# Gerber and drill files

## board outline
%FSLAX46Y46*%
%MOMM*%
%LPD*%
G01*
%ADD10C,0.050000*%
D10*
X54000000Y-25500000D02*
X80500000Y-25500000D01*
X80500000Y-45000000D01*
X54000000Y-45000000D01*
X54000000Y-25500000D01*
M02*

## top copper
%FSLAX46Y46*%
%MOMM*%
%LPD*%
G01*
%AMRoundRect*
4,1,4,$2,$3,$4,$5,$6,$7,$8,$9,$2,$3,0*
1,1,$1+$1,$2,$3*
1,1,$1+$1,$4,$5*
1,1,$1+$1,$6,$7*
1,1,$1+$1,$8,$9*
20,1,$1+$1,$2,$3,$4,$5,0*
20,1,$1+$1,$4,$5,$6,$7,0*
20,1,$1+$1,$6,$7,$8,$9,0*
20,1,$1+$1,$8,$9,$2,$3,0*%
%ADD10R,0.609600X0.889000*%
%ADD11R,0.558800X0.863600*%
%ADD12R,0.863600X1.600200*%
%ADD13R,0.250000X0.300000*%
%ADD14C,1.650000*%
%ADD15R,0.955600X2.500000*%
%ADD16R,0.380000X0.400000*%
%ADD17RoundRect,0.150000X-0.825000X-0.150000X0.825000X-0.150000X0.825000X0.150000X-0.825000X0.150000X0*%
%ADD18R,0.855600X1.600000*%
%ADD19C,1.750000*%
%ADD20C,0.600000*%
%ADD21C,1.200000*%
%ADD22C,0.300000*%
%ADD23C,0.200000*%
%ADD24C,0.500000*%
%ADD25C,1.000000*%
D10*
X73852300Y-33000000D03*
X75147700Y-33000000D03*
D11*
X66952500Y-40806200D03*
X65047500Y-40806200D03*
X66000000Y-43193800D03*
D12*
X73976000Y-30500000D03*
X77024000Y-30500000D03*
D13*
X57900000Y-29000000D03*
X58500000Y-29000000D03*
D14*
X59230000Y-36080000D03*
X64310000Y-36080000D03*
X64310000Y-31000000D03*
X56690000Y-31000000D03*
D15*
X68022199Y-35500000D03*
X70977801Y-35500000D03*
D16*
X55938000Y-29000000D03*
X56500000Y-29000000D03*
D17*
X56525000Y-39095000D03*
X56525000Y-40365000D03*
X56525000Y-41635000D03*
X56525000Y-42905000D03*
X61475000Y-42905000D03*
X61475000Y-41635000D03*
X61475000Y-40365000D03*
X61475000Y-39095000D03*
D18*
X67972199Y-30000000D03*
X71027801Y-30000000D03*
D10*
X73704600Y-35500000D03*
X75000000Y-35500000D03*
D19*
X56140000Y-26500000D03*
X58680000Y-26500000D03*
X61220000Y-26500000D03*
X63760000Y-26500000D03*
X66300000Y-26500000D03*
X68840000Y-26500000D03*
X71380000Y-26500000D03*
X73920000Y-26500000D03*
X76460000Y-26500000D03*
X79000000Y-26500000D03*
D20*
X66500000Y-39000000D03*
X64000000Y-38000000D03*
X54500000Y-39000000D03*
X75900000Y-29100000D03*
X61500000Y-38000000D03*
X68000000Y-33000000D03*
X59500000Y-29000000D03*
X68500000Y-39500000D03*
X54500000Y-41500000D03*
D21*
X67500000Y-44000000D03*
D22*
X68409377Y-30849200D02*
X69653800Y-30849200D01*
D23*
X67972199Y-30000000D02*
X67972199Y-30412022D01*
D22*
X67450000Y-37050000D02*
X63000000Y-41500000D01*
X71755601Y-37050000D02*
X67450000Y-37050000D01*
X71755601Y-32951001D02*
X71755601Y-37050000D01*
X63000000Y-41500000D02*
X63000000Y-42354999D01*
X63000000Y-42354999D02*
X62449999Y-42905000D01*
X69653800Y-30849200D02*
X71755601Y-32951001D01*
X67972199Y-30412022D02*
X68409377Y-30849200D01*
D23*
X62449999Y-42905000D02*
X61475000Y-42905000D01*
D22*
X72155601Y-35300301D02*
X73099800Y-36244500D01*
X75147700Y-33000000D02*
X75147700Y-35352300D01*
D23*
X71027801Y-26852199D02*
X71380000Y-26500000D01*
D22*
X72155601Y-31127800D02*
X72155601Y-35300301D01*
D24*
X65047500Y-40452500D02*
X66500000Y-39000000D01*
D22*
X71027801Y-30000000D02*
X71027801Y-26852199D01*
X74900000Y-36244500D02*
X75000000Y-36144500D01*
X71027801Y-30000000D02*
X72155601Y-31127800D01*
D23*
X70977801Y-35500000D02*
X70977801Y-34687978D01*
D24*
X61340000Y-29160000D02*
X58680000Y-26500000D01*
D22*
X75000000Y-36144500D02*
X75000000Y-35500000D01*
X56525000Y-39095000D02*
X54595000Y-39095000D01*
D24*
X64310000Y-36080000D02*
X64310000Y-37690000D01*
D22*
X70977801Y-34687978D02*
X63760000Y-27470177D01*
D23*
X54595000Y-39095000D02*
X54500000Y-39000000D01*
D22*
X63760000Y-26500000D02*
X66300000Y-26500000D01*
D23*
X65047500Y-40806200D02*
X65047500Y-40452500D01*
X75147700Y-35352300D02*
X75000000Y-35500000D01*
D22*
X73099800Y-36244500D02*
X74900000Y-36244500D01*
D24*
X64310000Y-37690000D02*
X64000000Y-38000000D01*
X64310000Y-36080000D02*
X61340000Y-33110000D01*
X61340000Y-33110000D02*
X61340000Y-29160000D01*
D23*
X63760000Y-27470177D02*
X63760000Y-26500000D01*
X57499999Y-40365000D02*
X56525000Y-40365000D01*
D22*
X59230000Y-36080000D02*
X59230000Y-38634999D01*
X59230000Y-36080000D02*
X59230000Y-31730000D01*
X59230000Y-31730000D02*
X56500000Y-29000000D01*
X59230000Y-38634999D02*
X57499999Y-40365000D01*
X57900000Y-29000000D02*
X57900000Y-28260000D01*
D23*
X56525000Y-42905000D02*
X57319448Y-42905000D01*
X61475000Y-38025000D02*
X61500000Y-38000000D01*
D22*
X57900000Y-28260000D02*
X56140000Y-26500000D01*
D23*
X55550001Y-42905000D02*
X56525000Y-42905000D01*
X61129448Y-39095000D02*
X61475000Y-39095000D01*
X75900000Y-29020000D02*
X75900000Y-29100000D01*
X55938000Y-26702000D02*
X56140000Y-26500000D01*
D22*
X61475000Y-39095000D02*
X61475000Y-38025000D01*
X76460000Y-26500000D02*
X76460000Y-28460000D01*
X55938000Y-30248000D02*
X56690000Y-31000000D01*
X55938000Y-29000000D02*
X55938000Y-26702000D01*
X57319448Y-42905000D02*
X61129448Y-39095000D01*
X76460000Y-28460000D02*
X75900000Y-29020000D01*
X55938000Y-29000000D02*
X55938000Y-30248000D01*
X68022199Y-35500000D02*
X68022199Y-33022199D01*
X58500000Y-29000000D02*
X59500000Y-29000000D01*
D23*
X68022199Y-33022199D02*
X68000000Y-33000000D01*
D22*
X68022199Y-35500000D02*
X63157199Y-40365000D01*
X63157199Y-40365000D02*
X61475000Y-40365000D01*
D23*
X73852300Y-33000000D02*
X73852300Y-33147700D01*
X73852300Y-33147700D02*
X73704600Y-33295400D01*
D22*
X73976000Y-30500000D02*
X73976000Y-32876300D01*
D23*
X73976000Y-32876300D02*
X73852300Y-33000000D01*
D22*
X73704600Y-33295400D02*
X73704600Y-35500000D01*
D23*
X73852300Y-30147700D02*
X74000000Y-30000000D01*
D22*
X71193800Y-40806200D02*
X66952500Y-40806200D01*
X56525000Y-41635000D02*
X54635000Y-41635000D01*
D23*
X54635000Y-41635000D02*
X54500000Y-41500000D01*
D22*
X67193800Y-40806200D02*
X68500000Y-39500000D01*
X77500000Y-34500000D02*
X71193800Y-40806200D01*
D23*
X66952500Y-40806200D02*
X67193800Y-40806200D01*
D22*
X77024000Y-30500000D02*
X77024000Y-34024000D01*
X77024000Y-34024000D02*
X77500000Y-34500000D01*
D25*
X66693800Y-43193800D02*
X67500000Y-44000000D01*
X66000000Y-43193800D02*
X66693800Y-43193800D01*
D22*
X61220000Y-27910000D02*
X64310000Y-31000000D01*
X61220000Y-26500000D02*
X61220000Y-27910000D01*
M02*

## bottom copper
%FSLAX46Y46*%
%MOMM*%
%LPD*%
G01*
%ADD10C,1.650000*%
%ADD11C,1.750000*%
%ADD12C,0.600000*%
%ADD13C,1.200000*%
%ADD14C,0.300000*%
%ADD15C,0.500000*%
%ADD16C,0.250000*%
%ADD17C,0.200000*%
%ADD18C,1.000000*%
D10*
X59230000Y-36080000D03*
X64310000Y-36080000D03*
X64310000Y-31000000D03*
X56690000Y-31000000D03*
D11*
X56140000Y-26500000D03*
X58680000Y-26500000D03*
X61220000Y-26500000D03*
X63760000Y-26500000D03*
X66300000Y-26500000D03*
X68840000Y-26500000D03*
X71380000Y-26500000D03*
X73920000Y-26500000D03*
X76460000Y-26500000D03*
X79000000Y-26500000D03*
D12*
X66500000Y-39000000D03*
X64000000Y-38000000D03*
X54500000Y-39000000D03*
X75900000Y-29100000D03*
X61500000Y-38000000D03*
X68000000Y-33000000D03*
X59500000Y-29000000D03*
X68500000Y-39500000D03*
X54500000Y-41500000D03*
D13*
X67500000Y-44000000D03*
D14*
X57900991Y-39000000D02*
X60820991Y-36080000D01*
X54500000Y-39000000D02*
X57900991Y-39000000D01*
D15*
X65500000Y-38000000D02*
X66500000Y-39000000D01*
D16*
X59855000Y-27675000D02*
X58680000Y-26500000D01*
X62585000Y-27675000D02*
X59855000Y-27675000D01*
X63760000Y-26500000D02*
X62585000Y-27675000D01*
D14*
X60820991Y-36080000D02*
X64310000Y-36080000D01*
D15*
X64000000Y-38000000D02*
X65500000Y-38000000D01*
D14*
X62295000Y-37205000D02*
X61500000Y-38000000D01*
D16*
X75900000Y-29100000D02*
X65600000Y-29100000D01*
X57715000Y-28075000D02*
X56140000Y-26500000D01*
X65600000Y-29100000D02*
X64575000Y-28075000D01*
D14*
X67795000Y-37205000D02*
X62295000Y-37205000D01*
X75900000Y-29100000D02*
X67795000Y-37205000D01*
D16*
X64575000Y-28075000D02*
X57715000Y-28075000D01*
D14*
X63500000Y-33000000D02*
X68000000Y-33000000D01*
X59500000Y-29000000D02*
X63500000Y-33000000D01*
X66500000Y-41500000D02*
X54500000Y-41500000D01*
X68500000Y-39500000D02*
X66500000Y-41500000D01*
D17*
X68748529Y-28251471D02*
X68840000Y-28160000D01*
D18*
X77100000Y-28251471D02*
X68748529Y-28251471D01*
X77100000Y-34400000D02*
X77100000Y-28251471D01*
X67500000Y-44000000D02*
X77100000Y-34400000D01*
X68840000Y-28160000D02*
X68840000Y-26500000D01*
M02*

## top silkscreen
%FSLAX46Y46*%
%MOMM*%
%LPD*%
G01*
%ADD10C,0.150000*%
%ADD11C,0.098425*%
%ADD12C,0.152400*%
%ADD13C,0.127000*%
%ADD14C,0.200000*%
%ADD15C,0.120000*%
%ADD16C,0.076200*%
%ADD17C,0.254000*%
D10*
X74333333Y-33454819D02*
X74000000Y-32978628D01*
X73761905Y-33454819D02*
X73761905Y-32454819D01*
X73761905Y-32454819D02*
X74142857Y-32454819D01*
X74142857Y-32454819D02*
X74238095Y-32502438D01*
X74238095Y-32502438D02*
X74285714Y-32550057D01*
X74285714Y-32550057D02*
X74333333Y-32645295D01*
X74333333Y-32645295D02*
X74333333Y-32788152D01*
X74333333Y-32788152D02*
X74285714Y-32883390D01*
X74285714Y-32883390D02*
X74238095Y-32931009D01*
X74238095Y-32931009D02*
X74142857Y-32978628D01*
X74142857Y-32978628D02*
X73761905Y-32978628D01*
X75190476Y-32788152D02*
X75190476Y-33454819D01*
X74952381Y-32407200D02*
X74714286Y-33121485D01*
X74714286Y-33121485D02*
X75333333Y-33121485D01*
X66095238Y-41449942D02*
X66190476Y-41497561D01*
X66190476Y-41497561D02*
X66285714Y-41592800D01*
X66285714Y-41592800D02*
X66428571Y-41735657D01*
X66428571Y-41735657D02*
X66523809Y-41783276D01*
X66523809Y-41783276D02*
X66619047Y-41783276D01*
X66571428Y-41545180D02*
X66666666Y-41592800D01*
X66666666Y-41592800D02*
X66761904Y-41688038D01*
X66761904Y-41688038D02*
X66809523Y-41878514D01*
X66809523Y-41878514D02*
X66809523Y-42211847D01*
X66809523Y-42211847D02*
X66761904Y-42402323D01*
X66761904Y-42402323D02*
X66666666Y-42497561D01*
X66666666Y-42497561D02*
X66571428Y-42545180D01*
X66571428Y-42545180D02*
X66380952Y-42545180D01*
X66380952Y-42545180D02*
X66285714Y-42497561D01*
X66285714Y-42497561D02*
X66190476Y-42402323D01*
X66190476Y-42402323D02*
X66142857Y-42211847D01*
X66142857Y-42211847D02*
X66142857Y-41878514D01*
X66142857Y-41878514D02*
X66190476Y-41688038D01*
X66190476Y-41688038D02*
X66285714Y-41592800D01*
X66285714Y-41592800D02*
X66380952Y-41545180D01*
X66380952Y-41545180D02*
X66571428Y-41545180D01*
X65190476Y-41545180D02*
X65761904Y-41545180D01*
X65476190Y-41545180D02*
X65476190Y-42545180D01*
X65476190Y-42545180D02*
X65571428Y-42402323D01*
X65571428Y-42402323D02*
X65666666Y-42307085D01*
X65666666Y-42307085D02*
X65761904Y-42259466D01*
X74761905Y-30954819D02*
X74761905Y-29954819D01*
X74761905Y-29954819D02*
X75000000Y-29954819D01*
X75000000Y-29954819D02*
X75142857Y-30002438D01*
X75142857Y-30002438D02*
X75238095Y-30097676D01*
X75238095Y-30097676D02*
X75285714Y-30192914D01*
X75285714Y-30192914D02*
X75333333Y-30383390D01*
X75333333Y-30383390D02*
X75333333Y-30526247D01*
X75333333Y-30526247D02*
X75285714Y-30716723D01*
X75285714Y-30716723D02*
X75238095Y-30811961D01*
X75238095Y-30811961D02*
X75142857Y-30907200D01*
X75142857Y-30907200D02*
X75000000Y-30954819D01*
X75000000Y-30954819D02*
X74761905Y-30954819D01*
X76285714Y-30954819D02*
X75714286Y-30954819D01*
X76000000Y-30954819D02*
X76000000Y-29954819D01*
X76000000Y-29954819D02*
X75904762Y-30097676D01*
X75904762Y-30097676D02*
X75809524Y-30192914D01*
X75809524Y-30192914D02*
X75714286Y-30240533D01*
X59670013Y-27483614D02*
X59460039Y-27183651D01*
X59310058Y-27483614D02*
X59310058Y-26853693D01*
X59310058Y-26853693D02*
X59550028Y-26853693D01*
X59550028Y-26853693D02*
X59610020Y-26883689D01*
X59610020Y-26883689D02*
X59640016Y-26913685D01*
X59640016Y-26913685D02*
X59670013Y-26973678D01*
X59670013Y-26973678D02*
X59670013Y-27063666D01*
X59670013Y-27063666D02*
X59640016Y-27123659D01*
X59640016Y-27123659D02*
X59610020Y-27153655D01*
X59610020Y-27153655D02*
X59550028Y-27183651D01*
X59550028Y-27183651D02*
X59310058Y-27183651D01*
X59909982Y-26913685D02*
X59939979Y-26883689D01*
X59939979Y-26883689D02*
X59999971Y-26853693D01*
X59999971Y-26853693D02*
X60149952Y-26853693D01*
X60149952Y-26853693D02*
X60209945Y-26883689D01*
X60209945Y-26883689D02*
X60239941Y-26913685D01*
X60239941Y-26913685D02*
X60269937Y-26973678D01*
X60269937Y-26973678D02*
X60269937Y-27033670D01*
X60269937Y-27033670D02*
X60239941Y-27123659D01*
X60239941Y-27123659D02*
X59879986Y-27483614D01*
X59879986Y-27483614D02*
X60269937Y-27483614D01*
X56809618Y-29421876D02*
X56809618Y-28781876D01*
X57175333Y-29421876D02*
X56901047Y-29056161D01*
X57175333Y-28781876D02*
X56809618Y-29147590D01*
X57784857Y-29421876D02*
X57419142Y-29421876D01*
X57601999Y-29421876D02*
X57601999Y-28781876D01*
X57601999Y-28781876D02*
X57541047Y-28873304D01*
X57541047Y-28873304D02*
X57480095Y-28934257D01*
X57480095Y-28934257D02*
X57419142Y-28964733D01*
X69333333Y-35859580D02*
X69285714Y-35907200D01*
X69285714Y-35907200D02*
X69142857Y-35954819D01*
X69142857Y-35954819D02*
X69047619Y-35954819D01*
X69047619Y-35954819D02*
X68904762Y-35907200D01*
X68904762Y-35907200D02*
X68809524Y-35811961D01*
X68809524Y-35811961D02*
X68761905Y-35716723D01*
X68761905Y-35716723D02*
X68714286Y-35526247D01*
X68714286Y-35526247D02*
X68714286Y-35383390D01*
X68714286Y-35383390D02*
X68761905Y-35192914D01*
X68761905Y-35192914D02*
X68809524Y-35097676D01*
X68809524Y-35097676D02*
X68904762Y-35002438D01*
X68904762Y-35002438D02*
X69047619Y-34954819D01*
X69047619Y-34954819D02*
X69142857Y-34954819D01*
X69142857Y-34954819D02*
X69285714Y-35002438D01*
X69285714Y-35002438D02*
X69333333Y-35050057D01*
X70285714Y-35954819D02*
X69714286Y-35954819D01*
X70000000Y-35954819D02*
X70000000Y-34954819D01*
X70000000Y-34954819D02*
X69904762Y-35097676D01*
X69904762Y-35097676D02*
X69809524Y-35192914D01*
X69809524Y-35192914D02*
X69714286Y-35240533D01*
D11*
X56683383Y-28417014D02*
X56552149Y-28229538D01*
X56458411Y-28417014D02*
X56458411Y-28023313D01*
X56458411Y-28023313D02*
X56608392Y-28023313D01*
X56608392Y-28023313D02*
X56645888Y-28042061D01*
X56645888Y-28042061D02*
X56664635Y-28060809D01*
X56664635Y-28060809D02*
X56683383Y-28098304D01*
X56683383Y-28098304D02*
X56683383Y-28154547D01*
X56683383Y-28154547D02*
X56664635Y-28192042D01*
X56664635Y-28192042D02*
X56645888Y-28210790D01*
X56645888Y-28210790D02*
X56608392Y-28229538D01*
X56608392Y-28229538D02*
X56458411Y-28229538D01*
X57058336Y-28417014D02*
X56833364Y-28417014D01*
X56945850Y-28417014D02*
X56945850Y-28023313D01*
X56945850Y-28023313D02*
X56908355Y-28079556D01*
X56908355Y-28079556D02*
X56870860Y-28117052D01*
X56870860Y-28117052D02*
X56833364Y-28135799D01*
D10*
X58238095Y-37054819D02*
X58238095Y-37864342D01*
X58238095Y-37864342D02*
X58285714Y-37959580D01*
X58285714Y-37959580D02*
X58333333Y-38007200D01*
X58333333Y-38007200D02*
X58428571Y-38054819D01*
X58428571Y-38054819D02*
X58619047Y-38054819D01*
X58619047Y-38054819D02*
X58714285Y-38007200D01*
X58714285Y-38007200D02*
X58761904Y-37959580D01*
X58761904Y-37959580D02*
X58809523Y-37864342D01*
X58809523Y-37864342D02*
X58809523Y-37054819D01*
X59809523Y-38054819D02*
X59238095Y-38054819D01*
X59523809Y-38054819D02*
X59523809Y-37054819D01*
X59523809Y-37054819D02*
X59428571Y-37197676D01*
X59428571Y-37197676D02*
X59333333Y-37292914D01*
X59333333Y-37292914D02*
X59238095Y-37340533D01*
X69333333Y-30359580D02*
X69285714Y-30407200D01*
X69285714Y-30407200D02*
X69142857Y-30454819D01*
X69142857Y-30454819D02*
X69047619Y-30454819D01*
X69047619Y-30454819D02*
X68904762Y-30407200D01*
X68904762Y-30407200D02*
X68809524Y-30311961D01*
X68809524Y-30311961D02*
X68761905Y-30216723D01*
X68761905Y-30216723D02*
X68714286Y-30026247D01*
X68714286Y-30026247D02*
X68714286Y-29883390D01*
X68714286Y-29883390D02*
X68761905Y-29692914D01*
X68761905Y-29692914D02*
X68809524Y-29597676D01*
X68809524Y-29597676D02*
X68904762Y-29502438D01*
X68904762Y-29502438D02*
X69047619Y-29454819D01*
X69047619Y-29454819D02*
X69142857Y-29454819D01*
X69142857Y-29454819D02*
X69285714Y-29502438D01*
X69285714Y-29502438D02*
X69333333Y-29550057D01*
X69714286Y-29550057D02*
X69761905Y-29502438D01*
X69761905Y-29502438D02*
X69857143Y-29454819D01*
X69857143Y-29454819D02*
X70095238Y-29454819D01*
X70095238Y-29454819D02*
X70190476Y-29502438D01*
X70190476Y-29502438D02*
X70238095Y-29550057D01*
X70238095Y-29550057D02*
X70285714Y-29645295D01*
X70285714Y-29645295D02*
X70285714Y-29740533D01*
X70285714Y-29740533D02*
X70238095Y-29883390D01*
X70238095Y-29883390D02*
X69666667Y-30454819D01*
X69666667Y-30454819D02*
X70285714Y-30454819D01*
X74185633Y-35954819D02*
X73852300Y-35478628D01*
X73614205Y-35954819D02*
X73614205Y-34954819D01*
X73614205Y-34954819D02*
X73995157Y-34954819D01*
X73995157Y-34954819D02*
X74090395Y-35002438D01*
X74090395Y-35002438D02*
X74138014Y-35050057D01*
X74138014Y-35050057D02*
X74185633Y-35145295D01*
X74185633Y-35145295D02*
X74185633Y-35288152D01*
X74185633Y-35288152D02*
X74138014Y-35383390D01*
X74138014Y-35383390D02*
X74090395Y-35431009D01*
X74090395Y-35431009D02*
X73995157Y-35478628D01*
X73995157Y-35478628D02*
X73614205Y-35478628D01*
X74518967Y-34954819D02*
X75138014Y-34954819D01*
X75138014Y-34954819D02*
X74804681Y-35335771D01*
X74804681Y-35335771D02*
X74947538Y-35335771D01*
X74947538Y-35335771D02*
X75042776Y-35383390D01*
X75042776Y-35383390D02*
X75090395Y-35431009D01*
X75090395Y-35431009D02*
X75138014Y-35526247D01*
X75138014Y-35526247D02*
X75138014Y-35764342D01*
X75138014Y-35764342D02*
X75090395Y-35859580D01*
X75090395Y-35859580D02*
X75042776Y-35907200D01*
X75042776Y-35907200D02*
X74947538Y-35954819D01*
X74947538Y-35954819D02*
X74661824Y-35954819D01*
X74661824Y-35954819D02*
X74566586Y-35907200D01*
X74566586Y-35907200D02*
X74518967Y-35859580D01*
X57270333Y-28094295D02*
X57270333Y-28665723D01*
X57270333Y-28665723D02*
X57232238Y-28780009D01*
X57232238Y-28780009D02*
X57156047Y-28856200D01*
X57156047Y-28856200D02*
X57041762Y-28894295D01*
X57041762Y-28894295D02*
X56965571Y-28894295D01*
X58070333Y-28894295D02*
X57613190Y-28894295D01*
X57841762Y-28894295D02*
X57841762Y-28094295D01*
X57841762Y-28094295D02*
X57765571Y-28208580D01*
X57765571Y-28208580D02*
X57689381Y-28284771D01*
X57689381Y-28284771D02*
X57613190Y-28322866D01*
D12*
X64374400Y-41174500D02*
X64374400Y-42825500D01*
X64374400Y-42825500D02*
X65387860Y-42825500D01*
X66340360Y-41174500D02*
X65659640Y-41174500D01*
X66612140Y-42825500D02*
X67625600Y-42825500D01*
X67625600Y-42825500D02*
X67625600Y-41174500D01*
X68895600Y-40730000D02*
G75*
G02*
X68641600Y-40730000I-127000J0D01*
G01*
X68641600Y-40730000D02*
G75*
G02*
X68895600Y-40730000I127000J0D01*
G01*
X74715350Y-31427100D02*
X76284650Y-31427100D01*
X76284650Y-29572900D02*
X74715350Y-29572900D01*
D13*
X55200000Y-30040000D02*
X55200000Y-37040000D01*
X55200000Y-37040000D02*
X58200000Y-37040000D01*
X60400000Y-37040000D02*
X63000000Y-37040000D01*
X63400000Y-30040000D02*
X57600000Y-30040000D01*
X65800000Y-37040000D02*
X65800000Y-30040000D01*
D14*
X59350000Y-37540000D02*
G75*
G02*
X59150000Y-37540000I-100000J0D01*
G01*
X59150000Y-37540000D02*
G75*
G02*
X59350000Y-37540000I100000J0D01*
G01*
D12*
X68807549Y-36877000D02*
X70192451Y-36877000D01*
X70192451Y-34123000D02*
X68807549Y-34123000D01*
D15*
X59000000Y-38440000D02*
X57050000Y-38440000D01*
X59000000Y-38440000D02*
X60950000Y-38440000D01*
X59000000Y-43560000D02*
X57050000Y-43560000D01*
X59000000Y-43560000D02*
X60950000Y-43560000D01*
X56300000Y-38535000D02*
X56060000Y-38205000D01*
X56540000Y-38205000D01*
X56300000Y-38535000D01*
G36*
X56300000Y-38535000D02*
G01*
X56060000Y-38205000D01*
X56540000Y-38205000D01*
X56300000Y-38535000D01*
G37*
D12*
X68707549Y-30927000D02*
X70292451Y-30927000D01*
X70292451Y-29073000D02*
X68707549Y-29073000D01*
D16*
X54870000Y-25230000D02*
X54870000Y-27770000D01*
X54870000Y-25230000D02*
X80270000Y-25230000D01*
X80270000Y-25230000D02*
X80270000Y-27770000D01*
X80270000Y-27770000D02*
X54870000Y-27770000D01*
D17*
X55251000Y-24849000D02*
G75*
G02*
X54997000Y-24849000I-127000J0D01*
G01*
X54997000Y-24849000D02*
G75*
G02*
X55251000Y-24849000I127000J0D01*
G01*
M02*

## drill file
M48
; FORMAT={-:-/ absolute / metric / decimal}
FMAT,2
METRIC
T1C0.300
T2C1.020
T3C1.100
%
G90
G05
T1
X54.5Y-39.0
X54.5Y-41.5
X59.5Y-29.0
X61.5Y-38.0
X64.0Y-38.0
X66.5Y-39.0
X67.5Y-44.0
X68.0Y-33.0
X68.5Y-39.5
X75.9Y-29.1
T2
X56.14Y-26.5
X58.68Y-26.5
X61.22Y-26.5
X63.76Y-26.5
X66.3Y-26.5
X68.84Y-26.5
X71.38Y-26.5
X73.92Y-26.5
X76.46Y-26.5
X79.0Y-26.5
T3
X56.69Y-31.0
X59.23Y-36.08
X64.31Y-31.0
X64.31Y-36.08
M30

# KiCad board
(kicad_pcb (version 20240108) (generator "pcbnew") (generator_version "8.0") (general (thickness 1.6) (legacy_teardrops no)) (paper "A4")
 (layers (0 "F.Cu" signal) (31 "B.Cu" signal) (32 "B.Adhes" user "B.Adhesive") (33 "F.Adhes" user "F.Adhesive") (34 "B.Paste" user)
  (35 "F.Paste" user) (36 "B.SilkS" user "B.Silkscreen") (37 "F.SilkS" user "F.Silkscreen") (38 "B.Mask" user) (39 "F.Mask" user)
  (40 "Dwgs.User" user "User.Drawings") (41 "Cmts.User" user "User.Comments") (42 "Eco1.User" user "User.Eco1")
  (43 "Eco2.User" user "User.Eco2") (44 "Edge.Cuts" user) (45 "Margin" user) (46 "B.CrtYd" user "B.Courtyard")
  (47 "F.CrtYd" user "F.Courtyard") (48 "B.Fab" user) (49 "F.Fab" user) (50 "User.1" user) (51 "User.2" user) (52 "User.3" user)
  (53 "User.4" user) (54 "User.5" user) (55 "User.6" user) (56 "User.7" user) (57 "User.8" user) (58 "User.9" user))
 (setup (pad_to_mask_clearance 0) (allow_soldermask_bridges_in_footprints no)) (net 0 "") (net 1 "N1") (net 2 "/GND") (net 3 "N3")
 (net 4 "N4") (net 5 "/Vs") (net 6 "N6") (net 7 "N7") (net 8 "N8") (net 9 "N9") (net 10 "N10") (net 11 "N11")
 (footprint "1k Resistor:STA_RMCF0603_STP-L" (layer "F.Cu") (at 74.5 33)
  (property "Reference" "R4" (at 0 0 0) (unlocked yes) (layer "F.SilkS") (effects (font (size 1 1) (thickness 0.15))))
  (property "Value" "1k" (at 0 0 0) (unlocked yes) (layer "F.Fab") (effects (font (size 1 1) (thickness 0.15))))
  (pad "1" smd rect (at -0.6477 0) (size 0.6096 0.889) (layers "F.Cu" "F.Paste" "F.Mask") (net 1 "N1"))
  (pad "2" smd rect (at 0.6477 0) (size 0.6096 0.889) (layers "F.Cu" "F.Paste" "F.Mask") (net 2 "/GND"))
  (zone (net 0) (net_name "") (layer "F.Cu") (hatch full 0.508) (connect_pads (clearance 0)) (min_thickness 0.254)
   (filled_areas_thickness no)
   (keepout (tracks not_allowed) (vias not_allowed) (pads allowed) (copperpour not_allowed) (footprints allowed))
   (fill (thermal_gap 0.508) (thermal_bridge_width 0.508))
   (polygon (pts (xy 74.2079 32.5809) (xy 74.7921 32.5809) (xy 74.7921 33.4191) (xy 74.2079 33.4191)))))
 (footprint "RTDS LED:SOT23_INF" (layer "F.Cu") (at 66 42 180)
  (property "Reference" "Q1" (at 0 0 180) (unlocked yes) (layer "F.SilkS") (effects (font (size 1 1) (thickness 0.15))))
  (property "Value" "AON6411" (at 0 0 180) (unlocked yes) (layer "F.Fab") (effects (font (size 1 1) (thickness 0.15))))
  (fp_line (start 1.6256 0.8255) (end 1.6256 -0.8255) (stroke (width 0.1524) (type solid)) (layer "F.SilkS"))
  (fp_line (start 1.6256 -0.8255) (end 0.61214 -0.8255) (stroke (width 0.1524) (type solid)) (layer "F.SilkS"))
  (fp_line (start -0.34036 0.8255) (end 0.34036 0.8255) (stroke (width 0.1524) (type solid)) (layer "F.SilkS"))
  (fp_line (start -0.61214 -0.8255) (end -1.6256 -0.8255) (stroke (width 0.1524) (type solid)) (layer "F.SilkS"))
  (fp_line (start -1.6256 -0.8255) (end -1.6256 0.8255) (stroke (width 0.1524) (type solid)) (layer "F.SilkS"))
  (fp_circle (center -2.7686 1.27) (end -2.6416 1.27) (stroke (width 0.1524) (type solid)) (fill none) (layer "F.SilkS"))
  (pad "1" smd rect (at -0.9525 1.1938 180) (size 0.5588 0.8636) (layers "F.Cu" "F.Paste" "F.Mask") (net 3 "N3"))
  (pad "2" smd rect (at 0.9525 1.1938 180) (size 0.5588 0.8636) (layers "F.Cu" "F.Paste" "F.Mask") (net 2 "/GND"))
  (pad "3" smd rect (at 0 -1.1938 180) (size 0.5588 0.8636) (layers "F.Cu" "F.Paste" "F.Mask") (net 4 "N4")))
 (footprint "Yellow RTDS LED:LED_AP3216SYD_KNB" (layer "F.Cu") (at 75.5 30.5)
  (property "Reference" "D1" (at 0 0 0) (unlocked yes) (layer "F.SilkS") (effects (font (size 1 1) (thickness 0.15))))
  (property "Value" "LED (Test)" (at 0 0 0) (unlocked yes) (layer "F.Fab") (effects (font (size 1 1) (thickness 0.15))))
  (fp_line (start -0.78465 0.9271) (end 0.78465 0.9271) (stroke (width 0.1524) (type solid)) (layer "F.SilkS"))
  (fp_line (start 0.78465 -0.9271) (end -0.78465 -0.9271) (stroke (width 0.1524) (type solid)) (layer "F.SilkS"))
  (pad "1" smd rect (at -1.524 0) (size 0.8636 1.6002) (layers "F.Cu" "F.Paste" "F.Mask") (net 1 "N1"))
  (pad "2" smd rect (at 1.524 0) (size 0.8636 1.6002) (layers "F.Cu" "F.Paste" "F.Mask") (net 3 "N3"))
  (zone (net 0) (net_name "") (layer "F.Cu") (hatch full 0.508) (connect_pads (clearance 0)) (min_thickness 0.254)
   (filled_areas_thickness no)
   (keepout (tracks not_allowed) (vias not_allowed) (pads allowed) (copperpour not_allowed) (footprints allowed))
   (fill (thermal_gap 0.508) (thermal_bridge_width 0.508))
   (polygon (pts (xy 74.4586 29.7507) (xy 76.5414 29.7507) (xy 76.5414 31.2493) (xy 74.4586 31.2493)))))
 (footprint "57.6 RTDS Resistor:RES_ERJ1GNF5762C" (layer "F.Cu") (at 58.2 29)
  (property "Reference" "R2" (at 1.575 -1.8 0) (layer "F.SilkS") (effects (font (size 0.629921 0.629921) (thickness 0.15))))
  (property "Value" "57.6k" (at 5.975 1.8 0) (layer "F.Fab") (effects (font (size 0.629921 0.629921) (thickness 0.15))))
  (pad "1" smd rect (at -0.3 0) (size 0.25 0.3) (layers "F.Cu" "F.Paste" "F.Mask") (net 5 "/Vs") (solder_mask_margin 0.102))
  (pad "2" smd rect (at 0.3 0) (size 0.25 0.3) (layers "F.Cu" "F.Paste" "F.Mask") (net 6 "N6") (solder_mask_margin 0.102)))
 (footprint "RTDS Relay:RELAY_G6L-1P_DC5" (layer "F.Cu") (at 60.5 33.54)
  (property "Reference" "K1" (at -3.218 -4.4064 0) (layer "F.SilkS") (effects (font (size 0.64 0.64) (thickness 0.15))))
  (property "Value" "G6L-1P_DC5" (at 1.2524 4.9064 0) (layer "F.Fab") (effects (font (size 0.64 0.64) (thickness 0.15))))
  (fp_line (start -5.3 -3.5) (end -5.3 3.5) (stroke (width 0.127) (type solid)) (layer "F.SilkS"))
  (fp_line (start -5.3 3.5) (end -2.3 3.5) (stroke (width 0.127) (type solid)) (layer "F.SilkS"))
  (fp_line (start -0.1 3.5) (end 2.5 3.5) (stroke (width 0.127) (type solid)) (layer "F.SilkS"))
  (fp_line (start 2.9 -3.5) (end -2.9 -3.5) (stroke (width 0.127) (type solid)) (layer "F.SilkS"))
  (fp_line (start 5.3 3.5) (end 5.3 -3.5) (stroke (width 0.127) (type solid)) (layer "F.SilkS"))
  (fp_circle (center -1.25 4) (end -1.15 4) (stroke (width 0.2) (type solid)) (fill none) (layer "F.SilkS"))
  (pad "2" thru_hole circle (at -1.27 2.54) (size 1.65 1.65) (drill 1.1) (layers "*.Cu" "*.Mask") (remove_unused_layers no) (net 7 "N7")
   (solder_mask_margin 0.102))
  (pad "4" thru_hole circle (at 3.81 2.54) (size 1.65 1.65) (drill 1.1) (layers "*.Cu" "*.Mask") (remove_unused_layers no) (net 2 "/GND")
   (solder_mask_margin 0.102))
  (pad "5" thru_hole circle (at 3.81 -2.54) (size 1.65 1.65) (drill 1.1) (layers "*.Cu" "*.Mask") (remove_unused_layers no) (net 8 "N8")
   (solder_mask_margin 0.102))
  (pad "8" thru_hole circle (at -3.81 -2.54) (size 1.65 1.65) (drill 1.1) (layers "*.Cu" "*.Mask") (remove_unused_layers no) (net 5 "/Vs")
   (solder_mask_margin 0.102)))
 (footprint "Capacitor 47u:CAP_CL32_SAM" (layer "F.Cu") (at 69.5 35.5)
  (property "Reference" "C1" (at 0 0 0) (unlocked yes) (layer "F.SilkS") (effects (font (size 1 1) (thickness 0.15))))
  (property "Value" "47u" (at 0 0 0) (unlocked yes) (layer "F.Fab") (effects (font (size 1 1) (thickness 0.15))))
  (fp_line (start -0.692451 1.377) (end 0.692451 1.377) (stroke (width 0.1524) (type solid)) (layer "F.SilkS"))
  (fp_line (start 0.692451 -1.377) (end -0.692451 -1.377) (stroke (width 0.1524) (type solid)) (layer "F.SilkS"))
  (pad "1" smd rect (at -1.477801 0) (size 0.9556 2.5) (layers "F.Cu" "F.Paste" "F.Mask") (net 6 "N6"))
  (pad "2" smd rect (at 1.477801 0) (size 0.9556 2.5) (layers "F.Cu" "F.Paste" "F.Mask") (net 2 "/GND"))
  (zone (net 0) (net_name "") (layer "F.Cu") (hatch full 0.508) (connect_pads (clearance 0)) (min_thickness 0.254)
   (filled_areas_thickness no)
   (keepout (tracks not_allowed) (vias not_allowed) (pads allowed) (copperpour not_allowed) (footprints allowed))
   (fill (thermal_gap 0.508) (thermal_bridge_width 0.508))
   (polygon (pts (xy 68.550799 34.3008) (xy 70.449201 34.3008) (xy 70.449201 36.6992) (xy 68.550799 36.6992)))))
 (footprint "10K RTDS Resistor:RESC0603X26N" (layer "F.Cu") (at 56.219 29)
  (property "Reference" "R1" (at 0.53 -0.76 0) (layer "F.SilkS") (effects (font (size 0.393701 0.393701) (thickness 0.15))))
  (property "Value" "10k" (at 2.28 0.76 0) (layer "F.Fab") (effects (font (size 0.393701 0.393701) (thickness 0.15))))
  (pad "1" smd rect (at -0.281 0) (size 0.38 0.4) (layers "F.Cu" "F.Paste" "F.Mask") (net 5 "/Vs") (solder_mask_margin 0.102))
  (pad "2" smd rect (at 0.281 0) (size 0.38 0.4) (layers "F.Cu" "F.Paste" "F.Mask") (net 7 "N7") (solder_mask_margin 0.102)))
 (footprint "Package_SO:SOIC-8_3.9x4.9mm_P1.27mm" (layer "F.Cu") (at 59 41)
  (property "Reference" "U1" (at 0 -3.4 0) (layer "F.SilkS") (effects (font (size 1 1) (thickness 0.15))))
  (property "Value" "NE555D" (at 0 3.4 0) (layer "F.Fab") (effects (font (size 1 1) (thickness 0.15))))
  (fp_line (start 0 -2.56) (end -1.95 -2.56) (stroke (width 0.12) (type solid)) (layer "F.SilkS"))
  (fp_line (start 0 -2.56) (end 1.95 -2.56) (stroke (width 0.12) (type solid)) (layer "F.SilkS"))
  (fp_line (start 0 2.56) (end -1.95 2.56) (stroke (width 0.12) (type solid)) (layer "F.SilkS"))
  (fp_line (start 0 2.56) (end 1.95 2.56) (stroke (width 0.12) (type solid)) (layer "F.SilkS"))
  (fp_poly
   (pts (xy -2.7 -2.465) (xy -2.94 -2.795) (xy -2.46 -2.795) (xy -2.7 -2.465)) (stroke (width 0.12) (type solid)) (fill solid)
   (layer "F.SilkS"))
  (pad "1" smd roundrect (at -2.475 -1.905) (size 1.95 0.6) (layers "F.Cu" "F.Paste" "F.Mask") (roundrect_rratio 0.25) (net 2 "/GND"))
  (pad "2" smd roundrect (at -2.475 -0.635) (size 1.95 0.6) (layers "F.Cu" "F.Paste" "F.Mask") (roundrect_rratio 0.25) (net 7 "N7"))
  (pad "3" smd roundrect (at -2.475 0.635) (size 1.95 0.6) (layers "F.Cu" "F.Paste" "F.Mask") (roundrect_rratio 0.25) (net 3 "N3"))
  (pad "4" smd roundrect (at -2.475 1.905) (size 1.95 0.6) (layers "F.Cu" "F.Paste" "F.Mask") (roundrect_rratio 0.25) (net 5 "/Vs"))
  (pad "5" smd roundrect (at 2.475 1.905) (size 1.95 0.6) (layers "F.Cu" "F.Paste" "F.Mask") (roundrect_rratio 0.25) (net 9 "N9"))
  (pad "6" smd roundrect (at 2.475 0.635) (size 1.95 0.6) (layers "F.Cu" "F.Paste" "F.Mask") (roundrect_rratio 0.25) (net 6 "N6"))
  (pad "7" smd roundrect (at 2.475 -0.635) (size 1.95 0.6) (layers "F.Cu" "F.Paste" "F.Mask") (roundrect_rratio 0.25) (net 6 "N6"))
  (pad "8" smd roundrect (at 2.475 -1.905) (size 1.95 0.6) (layers "F.Cu" "F.Paste" "F.Mask") (roundrect_rratio 0.25) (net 5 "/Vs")))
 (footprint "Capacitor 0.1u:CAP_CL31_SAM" (layer "F.Cu") (at 69.5 30)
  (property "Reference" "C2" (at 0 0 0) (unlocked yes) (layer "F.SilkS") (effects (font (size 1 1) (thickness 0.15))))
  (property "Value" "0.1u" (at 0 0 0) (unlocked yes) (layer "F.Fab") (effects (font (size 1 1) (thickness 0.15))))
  (fp_line (start -0.792451 0.927) (end 0.792451 0.927) (stroke (width 0.1524) (type solid)) (layer "F.SilkS"))
  (fp_line (start 0.792451 -0.927) (end -0.792451 -0.927) (stroke (width 0.1524) (type solid)) (layer "F.SilkS"))
  (pad "1" smd rect (at -1.527801 0) (size 0.8556 1.6) (layers "F.Cu" "F.Paste" "F.Mask") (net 9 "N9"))
  (pad "2" smd rect (at 1.527801 0) (size 0.8556 1.6) (layers "F.Cu" "F.Paste" "F.Mask") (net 2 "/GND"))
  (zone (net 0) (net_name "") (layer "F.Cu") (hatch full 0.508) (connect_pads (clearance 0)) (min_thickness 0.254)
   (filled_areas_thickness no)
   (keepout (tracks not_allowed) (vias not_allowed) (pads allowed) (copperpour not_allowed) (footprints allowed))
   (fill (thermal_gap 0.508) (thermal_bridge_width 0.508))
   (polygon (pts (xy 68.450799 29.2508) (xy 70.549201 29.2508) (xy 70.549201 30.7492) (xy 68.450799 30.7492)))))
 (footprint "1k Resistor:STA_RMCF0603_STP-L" (layer "F.Cu") (at 74.3523 35.5)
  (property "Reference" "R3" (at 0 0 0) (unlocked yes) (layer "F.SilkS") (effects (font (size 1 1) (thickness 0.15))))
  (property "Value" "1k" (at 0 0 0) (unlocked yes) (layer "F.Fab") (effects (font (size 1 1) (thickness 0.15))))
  (pad "1" smd rect (at -0.6477 0) (size 0.6096 0.889) (layers "F.Cu" "F.Paste" "F.Mask") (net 1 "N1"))
  (pad "2" smd rect (at 0.6477 0) (size 0.6096 0.889) (layers "F.Cu" "F.Paste" "F.Mask") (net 2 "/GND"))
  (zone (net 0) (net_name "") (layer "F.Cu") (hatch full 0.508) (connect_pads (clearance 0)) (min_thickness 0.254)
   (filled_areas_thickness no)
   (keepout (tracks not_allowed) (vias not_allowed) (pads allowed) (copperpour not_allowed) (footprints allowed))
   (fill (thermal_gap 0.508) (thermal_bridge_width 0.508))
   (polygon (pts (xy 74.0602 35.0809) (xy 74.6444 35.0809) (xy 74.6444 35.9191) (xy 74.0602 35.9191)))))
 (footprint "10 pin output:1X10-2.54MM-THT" (layer "F.Cu") (at 56.14 26.5)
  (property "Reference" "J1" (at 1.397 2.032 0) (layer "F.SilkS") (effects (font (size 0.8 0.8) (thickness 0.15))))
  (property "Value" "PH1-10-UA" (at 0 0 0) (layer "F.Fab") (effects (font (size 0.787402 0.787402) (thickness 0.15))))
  (fp_line (start -1.27 -1.27) (end -1.27 1.27) (stroke (width 0.0762) (type solid)) (layer "F.SilkS"))
  (fp_line (start -1.27 -1.27) (end 24.13 -1.27) (stroke (width 0.0762) (type solid)) (layer "F.SilkS"))
  (fp_line (start 24.13 -1.27) (end 24.13 1.27) (stroke (width 0.0762) (type solid)) (layer "F.SilkS"))
  (fp_line (start 24.13 1.27) (end -1.27 1.27) (stroke (width 0.0762) (type solid)) (layer "F.SilkS"))
  (fp_circle (center -1.016 -1.651) (end -0.762 -1.651) (stroke (width 0) (type solid)) (fill solid) (layer "F.SilkS"))
  (pad "1" thru_hole circle (at 0 0) (size 1.75 1.75) (drill 1.02) (layers "*.Cu" "*.Mask") (remove_unused_layers no) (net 5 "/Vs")
   (solder_mask_margin 0.102))
  (pad "2" thru_hole circle (at 2.54 0) (size 1.75 1.75) (drill 1.02) (layers "*.Cu" "*.Mask") (remove_unused_layers no) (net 2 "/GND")
   (solder_mask_margin 0.102))
  (pad "3" thru_hole circle (at 5.08 0) (size 1.75 1.75) (drill 1.02) (layers "*.Cu" "*.Mask") (remove_unused_layers no) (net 8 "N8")
   (solder_mask_margin 0.102))
  (pad "4" thru_hole circle (at 7.62 0) (size 1.75 1.75) (drill 1.02) (layers "*.Cu" "*.Mask") (remove_unused_layers no) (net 2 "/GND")
   (solder_mask_margin 0.102))
  (pad "5" thru_hole circle (at 10.16 0) (size 1.75 1.75) (drill 1.02) (layers "*.Cu" "*.Mask") (remove_unused_layers no) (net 2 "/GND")
   (solder_mask_margin 0.102))
  (pad "6" thru_hole circle (at 12.7 0) (size 1.75 1.75) (drill 1.02) (layers "*.Cu" "*.Mask") (remove_unused_layers no) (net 4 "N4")
   (solder_mask_margin 0.102))
  (pad "7" thru_hole circle (at 15.24 0) (size 1.75 1.75) (drill 1.02) (layers "*.Cu" "*.Mask") (remove_unused_layers no) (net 2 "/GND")
   (solder_mask_margin 0.102))
  (pad "8" thru_hole circle (at 17.78 0) (size 1.75 1.75) (drill 1.02) (layers "*.Cu" "*.Mask") (remove_unused_layers no) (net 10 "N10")
   (solder_mask_margin 0.102))
  (pad "9" thru_hole circle (at 20.32 0) (size 1.75 1.75) (drill 1.02) (layers "*.Cu" "*.Mask") (remove_unused_layers no) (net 5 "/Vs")
   (solder_mask_margin 0.102))
  (pad "10" thru_hole circle (at 22.86 0) (size 1.75 1.75) (drill 1.02) (layers "*.Cu" "*.Mask") (remove_unused_layers no) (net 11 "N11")
   (solder_mask_margin 0.102)))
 (gr_rect (start 54 25.5) (end 80.5 45) (stroke (width 0.05) (type default)) (fill none) (layer "Edge.Cuts"))
 (segment (start 68.409377 30.8492) (end 69.6538 30.8492) (width 0.3) (layer "F.Cu") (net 9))
 (segment (start 67.972199 30) (end 67.972199 30.412022) (width 0.2) (layer "F.Cu") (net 9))
 (segment (start 67.45 37.05) (end 63 41.5) (width 0.3) (layer "F.Cu") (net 9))
 (segment (start 71.755601 37.05) (end 67.45 37.05) (width 0.3) (layer "F.Cu") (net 9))
 (segment (start 71.755601 32.951001) (end 71.755601 37.05) (width 0.3) (layer "F.Cu") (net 9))
 (segment (start 63 41.5) (end 63 42.354999) (width 0.3) (layer "F.Cu") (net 9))
 (segment (start 63 42.354999) (end 62.449999 42.905) (width 0.3) (layer "F.Cu") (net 9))
 (segment (start 69.6538 30.8492) (end 71.755601 32.951001) (width 0.3) (layer "F.Cu") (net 9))
 (segment (start 67.972199 30.412022) (end 68.409377 30.8492) (width 0.3) (layer "F.Cu") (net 9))
 (segment (start 62.449999 42.905) (end 61.475 42.905) (width 0.2) (layer "F.Cu") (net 9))
 (segment (start 72.155601 35.300301) (end 73.0998 36.2445) (width 0.3) (layer "F.Cu") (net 2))
 (segment (start 75.1477 33) (end 75.1477 35.3523) (width 0.3) (layer "F.Cu") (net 2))
 (segment (start 71.027801 26.852199) (end 71.38 26.5) (width 0.2) (layer "F.Cu") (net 2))
 (segment (start 72.155601 31.1278) (end 72.155601 35.300301) (width 0.3) (layer "F.Cu") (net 2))
 (segment (start 65.0475 40.4525) (end 66.5 39) (width 0.5) (layer "F.Cu") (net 2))
 (segment (start 71.027801 30) (end 71.027801 26.852199) (width 0.3) (layer "F.Cu") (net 2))
 (segment (start 74.9 36.2445) (end 75 36.1445) (width 0.3) (layer "F.Cu") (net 2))
 (segment (start 71.027801 30) (end 72.155601 31.1278) (width 0.3) (layer "F.Cu") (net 2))
 (segment (start 70.977801 35.5) (end 70.977801 34.687978) (width 0.2) (layer "F.Cu") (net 2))
 (segment (start 61.34 29.16) (end 58.68 26.5) (width 0.5) (layer "F.Cu") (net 2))
 (segment (start 75 36.1445) (end 75 35.5) (width 0.3) (layer "F.Cu") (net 2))
 (segment (start 56.525 39.095) (end 54.595 39.095) (width 0.3) (layer "F.Cu") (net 2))
 (segment (start 64.31 36.08) (end 64.31 37.69) (width 0.5) (layer "F.Cu") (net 2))
 (segment (start 70.977801 34.687978) (end 63.76 27.470177) (width 0.3) (layer "F.Cu") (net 2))
 (segment (start 54.595 39.095) (end 54.5 39) (width 0.2) (layer "F.Cu") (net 2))
 (segment (start 63.76 26.5) (end 66.3 26.5) (width 0.3) (layer "F.Cu") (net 2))
 (segment (start 65.0475 40.8062) (end 65.0475 40.4525) (width 0.2) (layer "F.Cu") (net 2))
 (segment (start 75.1477 35.3523) (end 75 35.5) (width 0.2) (layer "F.Cu") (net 2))
 (segment (start 73.0998 36.2445) (end 74.9 36.2445) (width 0.3) (layer "F.Cu") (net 2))
 (segment (start 64.31 37.69) (end 64 38) (width 0.5) (layer "F.Cu") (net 2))
 (segment (start 64.31 36.08) (end 61.34 33.11) (width 0.5) (layer "F.Cu") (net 2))
 (segment (start 61.34 33.11) (end 61.34 29.16) (width 0.5) (layer "F.Cu") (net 2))
 (segment (start 63.76 27.470177) (end 63.76 26.5) (width 0.2) (layer "F.Cu") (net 2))
 (via (at 66.5 39) (size 0.6) (drill 0.3) (layers "F.Cu" "B.Cu") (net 2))
 (via (at 64 38) (size 0.6) (drill 0.3) (layers "F.Cu" "B.Cu") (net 2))
 (via (at 54.5 39) (size 0.6) (drill 0.3) (layers "F.Cu" "B.Cu") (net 2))
 (segment (start 57.900991 39) (end 60.820991 36.08) (width 0.3) (layer "B.Cu") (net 2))
 (segment (start 54.5 39) (end 57.900991 39) (width 0.3) (layer "B.Cu") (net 2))
 (segment (start 65.5 38) (end 66.5 39) (width 0.5) (layer "B.Cu") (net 2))
 (segment (start 59.855 27.675) (end 58.68 26.5) (width 0.25) (layer "B.Cu") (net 2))
 (segment (start 62.585 27.675) (end 59.855 27.675) (width 0.25) (layer "B.Cu") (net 2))
 (segment (start 63.76 26.5) (end 62.585 27.675) (width 0.25) (layer "B.Cu") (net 2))
 (segment (start 60.820991 36.08) (end 64.31 36.08) (width 0.3) (layer "B.Cu") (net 2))
 (segment (start 64 38) (end 65.5 38) (width 0.5) (layer "B.Cu") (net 2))
 (segment (start 57.499999 40.365) (end 56.525 40.365) (width 0.2) (layer "F.Cu") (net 7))
 (segment (start 59.23 36.08) (end 59.23 38.634999) (width 0.3) (layer "F.Cu") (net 7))
 (segment (start 59.23 36.08) (end 59.23 31.73) (width 0.3) (layer "F.Cu") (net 7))
 (segment (start 59.23 31.73) (end 56.5 29) (width 0.3) (layer "F.Cu") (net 7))
 (segment (start 59.23 38.634999) (end 57.499999 40.365) (width 0.3) (layer "F.Cu") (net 7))
 (segment (start 57.9 29) (end 57.9 28.26) (width 0.3) (layer "F.Cu") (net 5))
 (segment (start 56.525 42.905) (end 57.319448 42.905) (width 0.2) (layer "F.Cu") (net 5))
 (segment (start 61.475 38.025) (end 61.5 38) (width 0.2) (layer "F.Cu") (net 5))
 (segment (start 57.9 28.26) (end 56.14 26.5) (width 0.3) (layer "F.Cu") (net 5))
 (segment (start 55.550001 42.905) (end 56.525 42.905) (width 0.2) (layer "F.Cu") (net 5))
 (segment (start 61.129448 39.095) (end 61.475 39.095) (width 0.2) (layer "F.Cu") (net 5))
 (segment (start 75.9 29.02) (end 75.9 29.1) (width 0.2) (layer "F.Cu") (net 5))
 (segment (start 55.938 26.702) (end 56.14 26.5) (width 0.2) (layer "F.Cu") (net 5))
 (segment (start 61.475 39.095) (end 61.475 38.025) (width 0.3) (layer "F.Cu") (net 5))
 (segment (start 76.46 26.5) (end 76.46 28.46) (width 0.3) (layer "F.Cu") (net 5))
 (segment (start 55.938 30.248) (end 56.69 31) (width 0.3) (layer "F.Cu") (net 5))
 (segment (start 55.938 29) (end 55.938 26.702) (width 0.3) (layer "F.Cu") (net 5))
 (segment (start 57.319448 42.905) (end 61.129448 39.095) (width 0.3) (layer "F.Cu") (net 5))
 (segment (start 76.46 28.46) (end 75.9 29.02) (width 0.3) (layer "F.Cu") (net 5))
 (segment (start 55.938 29) (end 55.938 30.248) (width 0.3) (layer "F.Cu") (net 5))
 (via (at 75.9 29.1) (size 0.6) (drill 0.3) (layers "F.Cu" "B.Cu") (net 5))
 (via (at 61.5 38) (size 0.6) (drill 0.3) (layers "F.Cu" "B.Cu") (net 5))
 (segment (start 62.295 37.205) (end 61.5 38) (width 0.3) (layer "B.Cu") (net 5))
 (segment (start 75.9 29.1) (end 65.6 29.1) (width 0.25) (layer "B.Cu") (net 5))
 (segment (start 57.715 28.075) (end 56.14 26.5) (width 0.25) (layer "B.Cu") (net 5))
 (segment (start 65.6 29.1) (end 64.575 28.075) (width 0.25) (layer "B.Cu") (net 5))
 (segment (start 67.795 37.205) (end 62.295 37.205) (width 0.3) (layer "B.Cu") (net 5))
 (segment (start 75.9 29.1) (end 67.795 37.205) (width 0.3) (layer "B.Cu") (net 5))
 (segment (start 64.575 28.075) (end 57.715 28.075) (width 0.25) (layer "B.Cu") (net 5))
 (segment (start 68.022199 35.5) (end 68.022199 33.022199) (width 0.3) (layer "F.Cu") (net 6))
 (segment (start 58.5 29) (end 59.5 29) (width 0.3) (layer "F.Cu") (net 6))
 (segment (start 68.022199 33.022199) (end 68 33) (width 0.2) (layer "F.Cu") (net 6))
 (segment (start 68.022199 35.5) (end 63.157199 40.365) (width 0.3) (layer "F.Cu") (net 6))
 (segment (start 63.157199 40.365) (end 61.475 40.365) (width 0.3) (layer "F.Cu") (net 6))
 (via (at 68 33) (size 0.6) (drill 0.3) (layers "F.Cu" "B.Cu") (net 6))
 (via (at 59.5 29) (size 0.6) (drill 0.3) (layers "F.Cu" "B.Cu") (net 6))
 (segment (start 63.5 33) (end 68 33) (width 0.3) (layer "B.Cu") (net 6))
 (segment (start 59.5 29) (end 63.5 33) (width 0.3) (layer "B.Cu") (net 6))
 (segment (start 73.8523 33) (end 73.8523 33.1477) (width 0.2) (layer "F.Cu") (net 1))
 (segment (start 73.8523 33.1477) (end 73.7046 33.2954) (width 0.2) (layer "F.Cu") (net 1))
 (segment (start 73.976 30.5) (end 73.976 32.8763) (width 0.3) (layer "F.Cu") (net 1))
 (segment (start 73.976 32.8763) (end 73.8523 33) (width 0.2) (layer "F.Cu") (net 1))
 (segment (start 73.7046 33.2954) (end 73.7046 35.5) (width 0.3) (layer "F.Cu") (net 1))
 (segment (start 73.8523 30.1477) (end 74 30) (width 0.2) (layer "F.Cu") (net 1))
 (segment (start 71.1938 40.8062) (end 66.9525 40.8062) (width 0.3) (layer "F.Cu") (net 3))
 (segment (start 56.525 41.635) (end 54.635 41.635) (width 0.3) (layer "F.Cu") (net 3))
 (segment (start 54.635 41.635) (end 54.5 41.5) (width 0.2) (layer "F.Cu") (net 3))
 (segment (start 67.1938 40.8062) (end 68.5 39.5) (width 0.3) (layer "F.Cu") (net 3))
 (segment (start 77.5 34.5) (end 71.1938 40.8062) (width 0.3) (layer "F.Cu") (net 3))
 (segment (start 66.9525 40.8062) (end 67.1938 40.8062) (width 0.2) (layer "F.Cu") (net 3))
 (segment (start 77.024 30.5) (end 77.024 34.024) (width 0.3) (layer "F.Cu") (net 3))
 (segment (start 77.024 34.024) (end 77.5 34.5) (width 0.3) (layer "F.Cu") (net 3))
 (via (at 68.5 39.5) (size 0.6) (drill 0.3) (layers "F.Cu" "B.Cu") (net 3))
 (via (at 54.5 41.5) (size 0.6) (drill 0.3) (layers "F.Cu" "B.Cu") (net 3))
 (segment (start 66.5 41.5) (end 54.5 41.5) (width 0.3) (layer "B.Cu") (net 3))
 (segment (start 68.5 39.5) (end 66.5 41.5) (width 0.3) (layer "B.Cu") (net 3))
 (segment (start 66.6938 43.1938) (end 67.5 44) (width 1) (layer "F.Cu") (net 4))
 (segment (start 66 43.1938) (end 66.6938 43.1938) (width 1) (layer "F.Cu") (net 4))
 (via (at 67.5 44) (size 1.2) (drill 0.3) (layers "F.Cu" "B.Cu") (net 4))
 (segment (start 68.748529 28.251471) (end 68.84 28.16) (width 0.2) (layer "B.Cu") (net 4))
 (segment (start 77.1 28.251471) (end 68.748529 28.251471) (width 1) (layer "B.Cu") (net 4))
 (segment (start 77.1 34.4) (end 77.1 28.251471) (width 1) (layer "B.Cu") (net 4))
 (segment (start 67.5 44) (end 77.1 34.4) (width 1) (layer "B.Cu") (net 4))
 (segment (start 68.84 28.16) (end 68.84 26.5) (width 1) (layer "B.Cu") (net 4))
 (segment (start 61.22 27.91) (end 64.31 31) (width 0.3) (layer "F.Cu") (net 8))
 (segment (start 61.22 26.5) (end 61.22 27.91) (width 0.3) (layer "F.Cu") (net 8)))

